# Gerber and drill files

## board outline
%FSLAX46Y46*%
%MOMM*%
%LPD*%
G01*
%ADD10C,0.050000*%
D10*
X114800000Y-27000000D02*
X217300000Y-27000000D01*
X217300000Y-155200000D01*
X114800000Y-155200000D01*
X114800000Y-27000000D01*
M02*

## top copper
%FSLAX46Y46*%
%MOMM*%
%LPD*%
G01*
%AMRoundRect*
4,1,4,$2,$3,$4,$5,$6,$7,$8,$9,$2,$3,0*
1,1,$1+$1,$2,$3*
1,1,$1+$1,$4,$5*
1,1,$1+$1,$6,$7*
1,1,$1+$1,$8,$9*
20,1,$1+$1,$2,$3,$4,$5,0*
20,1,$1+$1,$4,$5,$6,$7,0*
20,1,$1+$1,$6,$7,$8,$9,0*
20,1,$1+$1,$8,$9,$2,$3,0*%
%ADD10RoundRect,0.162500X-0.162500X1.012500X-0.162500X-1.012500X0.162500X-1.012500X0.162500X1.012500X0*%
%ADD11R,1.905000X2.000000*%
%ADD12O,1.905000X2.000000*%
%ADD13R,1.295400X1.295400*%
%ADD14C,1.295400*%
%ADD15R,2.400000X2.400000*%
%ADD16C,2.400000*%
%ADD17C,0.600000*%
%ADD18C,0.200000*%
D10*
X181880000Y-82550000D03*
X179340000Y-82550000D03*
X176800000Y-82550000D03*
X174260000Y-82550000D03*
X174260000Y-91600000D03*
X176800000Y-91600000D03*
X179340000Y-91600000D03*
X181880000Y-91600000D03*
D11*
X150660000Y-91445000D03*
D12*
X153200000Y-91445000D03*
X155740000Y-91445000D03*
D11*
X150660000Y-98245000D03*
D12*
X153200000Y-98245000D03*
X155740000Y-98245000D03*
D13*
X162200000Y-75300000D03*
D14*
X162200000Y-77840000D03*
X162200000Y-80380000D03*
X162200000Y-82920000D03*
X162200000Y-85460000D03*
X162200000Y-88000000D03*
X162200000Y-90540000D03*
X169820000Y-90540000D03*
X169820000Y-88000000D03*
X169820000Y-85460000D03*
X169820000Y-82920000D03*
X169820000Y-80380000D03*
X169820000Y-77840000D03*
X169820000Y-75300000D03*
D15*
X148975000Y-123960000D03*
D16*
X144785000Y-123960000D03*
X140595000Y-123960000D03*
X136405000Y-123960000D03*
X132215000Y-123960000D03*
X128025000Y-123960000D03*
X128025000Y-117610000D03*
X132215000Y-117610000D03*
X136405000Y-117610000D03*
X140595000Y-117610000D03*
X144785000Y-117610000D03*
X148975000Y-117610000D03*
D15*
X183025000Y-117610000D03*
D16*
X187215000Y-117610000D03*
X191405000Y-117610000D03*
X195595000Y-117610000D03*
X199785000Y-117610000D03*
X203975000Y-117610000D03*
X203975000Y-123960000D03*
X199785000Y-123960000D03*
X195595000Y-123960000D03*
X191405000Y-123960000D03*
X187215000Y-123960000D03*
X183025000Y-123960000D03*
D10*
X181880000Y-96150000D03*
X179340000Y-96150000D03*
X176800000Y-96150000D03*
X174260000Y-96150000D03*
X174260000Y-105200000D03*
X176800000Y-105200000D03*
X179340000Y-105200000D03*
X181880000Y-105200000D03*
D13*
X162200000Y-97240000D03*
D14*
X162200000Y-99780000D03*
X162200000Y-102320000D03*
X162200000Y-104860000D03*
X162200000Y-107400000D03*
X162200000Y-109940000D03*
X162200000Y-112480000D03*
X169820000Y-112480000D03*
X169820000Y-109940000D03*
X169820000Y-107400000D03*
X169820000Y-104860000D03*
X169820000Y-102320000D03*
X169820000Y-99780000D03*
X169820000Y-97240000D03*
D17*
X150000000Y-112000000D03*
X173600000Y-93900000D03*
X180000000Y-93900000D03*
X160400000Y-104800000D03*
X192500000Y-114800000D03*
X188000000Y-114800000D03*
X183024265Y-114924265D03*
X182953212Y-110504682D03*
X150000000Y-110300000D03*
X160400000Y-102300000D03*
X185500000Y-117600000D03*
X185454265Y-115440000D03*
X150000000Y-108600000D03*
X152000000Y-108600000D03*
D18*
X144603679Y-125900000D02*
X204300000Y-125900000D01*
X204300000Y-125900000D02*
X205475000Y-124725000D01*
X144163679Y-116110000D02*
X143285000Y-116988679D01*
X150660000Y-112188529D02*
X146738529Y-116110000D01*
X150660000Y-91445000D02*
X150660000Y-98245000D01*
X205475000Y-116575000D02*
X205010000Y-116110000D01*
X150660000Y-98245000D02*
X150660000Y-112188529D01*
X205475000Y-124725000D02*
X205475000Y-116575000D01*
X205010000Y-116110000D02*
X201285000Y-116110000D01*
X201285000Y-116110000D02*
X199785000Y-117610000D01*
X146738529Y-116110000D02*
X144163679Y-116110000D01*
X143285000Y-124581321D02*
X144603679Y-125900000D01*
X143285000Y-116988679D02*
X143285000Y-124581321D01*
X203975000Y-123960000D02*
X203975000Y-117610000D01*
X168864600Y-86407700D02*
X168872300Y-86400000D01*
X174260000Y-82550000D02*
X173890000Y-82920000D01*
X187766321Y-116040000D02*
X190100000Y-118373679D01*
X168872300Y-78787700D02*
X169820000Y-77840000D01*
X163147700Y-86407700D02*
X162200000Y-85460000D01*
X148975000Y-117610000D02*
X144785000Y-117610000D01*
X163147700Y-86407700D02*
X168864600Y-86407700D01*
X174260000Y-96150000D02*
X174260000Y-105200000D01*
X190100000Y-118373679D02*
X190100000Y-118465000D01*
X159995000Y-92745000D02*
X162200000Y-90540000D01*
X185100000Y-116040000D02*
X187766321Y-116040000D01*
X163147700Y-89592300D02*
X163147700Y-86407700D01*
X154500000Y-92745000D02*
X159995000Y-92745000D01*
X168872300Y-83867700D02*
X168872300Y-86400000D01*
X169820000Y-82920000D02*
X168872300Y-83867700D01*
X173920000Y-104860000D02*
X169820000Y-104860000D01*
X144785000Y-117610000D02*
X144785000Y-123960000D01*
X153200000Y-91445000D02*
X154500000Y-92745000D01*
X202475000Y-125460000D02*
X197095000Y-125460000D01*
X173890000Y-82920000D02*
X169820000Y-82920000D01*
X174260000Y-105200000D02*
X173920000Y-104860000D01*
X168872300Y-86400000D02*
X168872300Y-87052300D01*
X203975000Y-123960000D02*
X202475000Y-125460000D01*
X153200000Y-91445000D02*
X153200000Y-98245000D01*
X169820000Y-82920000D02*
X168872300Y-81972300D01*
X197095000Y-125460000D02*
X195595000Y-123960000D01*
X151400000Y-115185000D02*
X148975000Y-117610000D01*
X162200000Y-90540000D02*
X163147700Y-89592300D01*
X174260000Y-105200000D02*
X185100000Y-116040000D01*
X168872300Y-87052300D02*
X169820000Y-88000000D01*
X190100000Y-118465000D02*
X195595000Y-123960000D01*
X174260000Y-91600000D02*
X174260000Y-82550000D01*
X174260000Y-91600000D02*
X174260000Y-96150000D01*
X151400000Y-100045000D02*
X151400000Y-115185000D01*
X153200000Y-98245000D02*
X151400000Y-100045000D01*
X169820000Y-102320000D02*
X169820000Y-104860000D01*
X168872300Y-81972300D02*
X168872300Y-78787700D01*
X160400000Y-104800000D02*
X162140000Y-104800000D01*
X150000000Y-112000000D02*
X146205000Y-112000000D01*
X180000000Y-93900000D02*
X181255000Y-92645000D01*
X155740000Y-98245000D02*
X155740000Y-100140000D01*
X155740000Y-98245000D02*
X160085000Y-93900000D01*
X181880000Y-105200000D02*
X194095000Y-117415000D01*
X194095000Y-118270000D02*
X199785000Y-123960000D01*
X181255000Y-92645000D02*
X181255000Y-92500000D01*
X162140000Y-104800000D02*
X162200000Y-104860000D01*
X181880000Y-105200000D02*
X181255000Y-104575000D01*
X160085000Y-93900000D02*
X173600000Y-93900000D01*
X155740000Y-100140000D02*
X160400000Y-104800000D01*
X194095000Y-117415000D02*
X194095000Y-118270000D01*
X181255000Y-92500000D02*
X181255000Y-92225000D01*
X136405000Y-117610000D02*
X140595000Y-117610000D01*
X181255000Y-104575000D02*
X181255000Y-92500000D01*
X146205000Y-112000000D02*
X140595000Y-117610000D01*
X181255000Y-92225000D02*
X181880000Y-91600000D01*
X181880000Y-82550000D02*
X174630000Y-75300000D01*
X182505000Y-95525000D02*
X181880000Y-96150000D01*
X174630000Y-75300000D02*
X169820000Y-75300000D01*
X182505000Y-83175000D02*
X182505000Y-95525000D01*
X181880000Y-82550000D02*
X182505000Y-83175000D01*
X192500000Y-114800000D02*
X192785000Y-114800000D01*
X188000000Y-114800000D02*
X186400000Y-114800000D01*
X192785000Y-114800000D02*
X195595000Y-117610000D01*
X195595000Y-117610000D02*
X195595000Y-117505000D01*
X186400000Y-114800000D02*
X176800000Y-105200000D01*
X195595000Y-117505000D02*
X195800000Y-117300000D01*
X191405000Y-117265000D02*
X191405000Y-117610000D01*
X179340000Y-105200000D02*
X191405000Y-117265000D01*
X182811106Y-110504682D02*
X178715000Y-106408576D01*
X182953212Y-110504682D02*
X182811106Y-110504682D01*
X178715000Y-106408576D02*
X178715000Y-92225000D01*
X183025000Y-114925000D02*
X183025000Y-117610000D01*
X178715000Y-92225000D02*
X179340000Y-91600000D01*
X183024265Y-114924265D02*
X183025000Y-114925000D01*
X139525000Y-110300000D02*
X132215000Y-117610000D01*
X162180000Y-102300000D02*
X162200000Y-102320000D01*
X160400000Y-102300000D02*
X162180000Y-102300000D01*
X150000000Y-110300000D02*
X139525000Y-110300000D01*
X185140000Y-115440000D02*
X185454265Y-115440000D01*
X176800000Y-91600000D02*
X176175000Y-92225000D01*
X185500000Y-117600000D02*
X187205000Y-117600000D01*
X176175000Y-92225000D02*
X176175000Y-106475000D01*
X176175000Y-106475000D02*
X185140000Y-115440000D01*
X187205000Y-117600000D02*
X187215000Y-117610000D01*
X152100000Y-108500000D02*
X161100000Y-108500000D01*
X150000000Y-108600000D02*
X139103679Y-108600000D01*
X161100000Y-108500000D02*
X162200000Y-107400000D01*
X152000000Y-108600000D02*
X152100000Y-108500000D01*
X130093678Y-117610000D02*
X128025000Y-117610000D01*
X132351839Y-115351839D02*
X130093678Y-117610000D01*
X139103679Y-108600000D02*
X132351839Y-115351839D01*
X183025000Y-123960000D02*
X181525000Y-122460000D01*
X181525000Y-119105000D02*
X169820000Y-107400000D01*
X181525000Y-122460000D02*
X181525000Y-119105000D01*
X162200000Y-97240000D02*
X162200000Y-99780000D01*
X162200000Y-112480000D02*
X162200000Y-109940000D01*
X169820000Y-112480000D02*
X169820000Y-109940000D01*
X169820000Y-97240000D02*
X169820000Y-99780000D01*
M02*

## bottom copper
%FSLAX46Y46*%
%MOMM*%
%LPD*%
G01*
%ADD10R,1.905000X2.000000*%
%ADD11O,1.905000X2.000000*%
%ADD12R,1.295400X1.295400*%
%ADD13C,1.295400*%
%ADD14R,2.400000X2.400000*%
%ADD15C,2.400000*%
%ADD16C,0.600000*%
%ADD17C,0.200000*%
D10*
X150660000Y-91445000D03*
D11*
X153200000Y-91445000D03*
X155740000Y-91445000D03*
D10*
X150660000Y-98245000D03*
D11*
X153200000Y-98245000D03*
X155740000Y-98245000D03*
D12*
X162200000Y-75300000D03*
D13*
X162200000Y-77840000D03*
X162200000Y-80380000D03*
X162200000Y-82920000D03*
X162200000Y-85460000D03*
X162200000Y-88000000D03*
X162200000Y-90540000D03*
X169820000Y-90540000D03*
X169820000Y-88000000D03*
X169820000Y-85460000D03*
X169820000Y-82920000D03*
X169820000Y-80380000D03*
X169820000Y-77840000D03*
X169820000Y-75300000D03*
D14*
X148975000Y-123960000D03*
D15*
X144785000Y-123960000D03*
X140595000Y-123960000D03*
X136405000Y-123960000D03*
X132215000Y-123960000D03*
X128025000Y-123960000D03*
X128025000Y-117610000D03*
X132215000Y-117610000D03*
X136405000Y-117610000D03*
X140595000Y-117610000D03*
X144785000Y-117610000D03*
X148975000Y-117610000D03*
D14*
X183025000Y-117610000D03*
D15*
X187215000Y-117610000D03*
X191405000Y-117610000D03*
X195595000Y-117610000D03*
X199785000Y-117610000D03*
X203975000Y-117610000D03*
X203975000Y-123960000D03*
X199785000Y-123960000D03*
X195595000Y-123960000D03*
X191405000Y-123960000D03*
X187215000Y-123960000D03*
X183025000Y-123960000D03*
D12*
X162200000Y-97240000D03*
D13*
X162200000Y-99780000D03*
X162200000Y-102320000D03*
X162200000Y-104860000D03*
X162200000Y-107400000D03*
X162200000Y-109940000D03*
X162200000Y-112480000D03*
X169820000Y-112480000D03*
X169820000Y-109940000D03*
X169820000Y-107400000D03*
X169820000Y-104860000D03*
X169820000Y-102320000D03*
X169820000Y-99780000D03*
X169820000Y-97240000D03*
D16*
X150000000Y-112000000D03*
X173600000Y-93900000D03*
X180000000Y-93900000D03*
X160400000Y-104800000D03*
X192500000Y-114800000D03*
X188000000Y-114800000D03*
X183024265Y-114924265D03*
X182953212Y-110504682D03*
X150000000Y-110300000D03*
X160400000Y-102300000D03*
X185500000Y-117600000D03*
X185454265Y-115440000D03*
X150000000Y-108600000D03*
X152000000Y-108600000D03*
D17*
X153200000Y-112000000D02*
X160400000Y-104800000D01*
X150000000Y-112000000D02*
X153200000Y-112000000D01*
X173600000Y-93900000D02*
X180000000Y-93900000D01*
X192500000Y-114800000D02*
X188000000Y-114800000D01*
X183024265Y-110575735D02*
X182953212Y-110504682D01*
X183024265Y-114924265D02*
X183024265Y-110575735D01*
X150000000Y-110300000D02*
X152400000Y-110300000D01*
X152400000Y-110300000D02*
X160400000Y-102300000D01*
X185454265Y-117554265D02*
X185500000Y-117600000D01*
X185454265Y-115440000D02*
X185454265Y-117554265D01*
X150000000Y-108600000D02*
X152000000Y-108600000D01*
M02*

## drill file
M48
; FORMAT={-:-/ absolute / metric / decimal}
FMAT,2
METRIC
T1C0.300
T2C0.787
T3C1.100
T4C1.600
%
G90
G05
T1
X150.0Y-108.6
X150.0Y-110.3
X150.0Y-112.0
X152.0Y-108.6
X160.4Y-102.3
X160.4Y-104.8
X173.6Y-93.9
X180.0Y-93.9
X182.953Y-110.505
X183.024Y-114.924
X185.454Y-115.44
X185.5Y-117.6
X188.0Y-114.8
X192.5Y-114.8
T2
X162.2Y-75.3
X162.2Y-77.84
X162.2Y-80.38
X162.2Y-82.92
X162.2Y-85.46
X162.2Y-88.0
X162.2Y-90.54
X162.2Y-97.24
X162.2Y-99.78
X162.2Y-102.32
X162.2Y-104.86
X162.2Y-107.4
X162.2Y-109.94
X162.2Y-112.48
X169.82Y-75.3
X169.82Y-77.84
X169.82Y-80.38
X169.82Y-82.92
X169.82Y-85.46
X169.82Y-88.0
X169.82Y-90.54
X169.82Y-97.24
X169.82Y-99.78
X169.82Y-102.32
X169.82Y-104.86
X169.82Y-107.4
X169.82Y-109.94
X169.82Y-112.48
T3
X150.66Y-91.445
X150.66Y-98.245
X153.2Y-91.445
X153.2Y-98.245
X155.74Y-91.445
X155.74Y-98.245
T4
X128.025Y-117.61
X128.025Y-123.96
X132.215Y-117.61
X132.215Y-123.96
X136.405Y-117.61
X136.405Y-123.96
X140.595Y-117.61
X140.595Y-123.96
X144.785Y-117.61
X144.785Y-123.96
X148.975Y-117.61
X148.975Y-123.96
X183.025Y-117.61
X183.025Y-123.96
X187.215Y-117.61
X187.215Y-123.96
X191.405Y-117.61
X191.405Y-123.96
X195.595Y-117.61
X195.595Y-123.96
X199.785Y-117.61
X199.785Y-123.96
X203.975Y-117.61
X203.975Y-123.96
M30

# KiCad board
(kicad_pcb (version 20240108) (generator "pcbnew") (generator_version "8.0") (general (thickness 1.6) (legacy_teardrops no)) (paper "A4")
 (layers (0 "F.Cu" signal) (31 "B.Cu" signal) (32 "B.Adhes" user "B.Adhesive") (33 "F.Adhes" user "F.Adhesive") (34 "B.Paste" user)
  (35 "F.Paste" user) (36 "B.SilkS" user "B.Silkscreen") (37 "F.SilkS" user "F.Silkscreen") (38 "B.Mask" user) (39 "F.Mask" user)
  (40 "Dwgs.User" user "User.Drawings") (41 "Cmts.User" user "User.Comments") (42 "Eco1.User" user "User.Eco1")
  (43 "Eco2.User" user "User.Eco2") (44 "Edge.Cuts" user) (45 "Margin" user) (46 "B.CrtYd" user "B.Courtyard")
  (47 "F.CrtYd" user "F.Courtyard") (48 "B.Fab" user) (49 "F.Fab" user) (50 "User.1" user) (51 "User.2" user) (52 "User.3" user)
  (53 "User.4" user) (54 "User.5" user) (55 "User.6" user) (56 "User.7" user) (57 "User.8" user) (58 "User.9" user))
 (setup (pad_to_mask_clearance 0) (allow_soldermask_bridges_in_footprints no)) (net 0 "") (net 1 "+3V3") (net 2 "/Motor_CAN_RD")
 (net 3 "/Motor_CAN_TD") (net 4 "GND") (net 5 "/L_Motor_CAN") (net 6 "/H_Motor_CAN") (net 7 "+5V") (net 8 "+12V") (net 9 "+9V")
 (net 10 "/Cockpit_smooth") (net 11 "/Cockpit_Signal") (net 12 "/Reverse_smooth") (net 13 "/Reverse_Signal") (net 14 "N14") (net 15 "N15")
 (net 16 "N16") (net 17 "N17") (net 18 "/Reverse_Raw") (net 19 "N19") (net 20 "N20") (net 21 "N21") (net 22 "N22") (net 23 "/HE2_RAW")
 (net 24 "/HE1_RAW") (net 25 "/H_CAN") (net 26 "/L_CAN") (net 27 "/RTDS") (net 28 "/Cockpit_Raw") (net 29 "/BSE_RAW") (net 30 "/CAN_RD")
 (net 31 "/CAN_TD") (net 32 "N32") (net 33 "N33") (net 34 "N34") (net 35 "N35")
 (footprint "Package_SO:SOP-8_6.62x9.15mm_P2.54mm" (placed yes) (layer "F.Cu") (at 178.07 87.075 -90)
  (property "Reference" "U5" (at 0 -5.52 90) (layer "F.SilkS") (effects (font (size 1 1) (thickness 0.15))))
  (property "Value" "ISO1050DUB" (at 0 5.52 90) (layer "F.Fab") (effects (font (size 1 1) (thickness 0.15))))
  (pad "1" smd roundrect (at -4.525 -3.81 270) (size 2.35 0.65) (layers "F.Cu" "F.Paste" "F.Mask") (roundrect_rratio 0.25) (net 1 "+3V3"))
  (pad "2" smd roundrect (at -4.525 -1.27 270) (size 2.35 0.65) (layers "F.Cu" "F.Paste" "F.Mask") (roundrect_rratio 0.25)
   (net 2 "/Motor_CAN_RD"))
  (pad "3" smd roundrect (at -4.525 1.27 270) (size 2.35 0.65) (layers "F.Cu" "F.Paste" "F.Mask") (roundrect_rratio 0.25)
   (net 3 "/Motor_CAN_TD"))
  (pad "4" smd roundrect (at -4.525 3.81 270) (size 2.35 0.65) (layers "F.Cu" "F.Paste" "F.Mask") (roundrect_rratio 0.25) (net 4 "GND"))
  (pad "5" smd roundrect (at 4.525 3.81 270) (size 2.35 0.65) (layers "F.Cu" "F.Paste" "F.Mask") (roundrect_rratio 0.25) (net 4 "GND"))
  (pad "6" smd roundrect (at 4.525 1.27 270) (size 2.35 0.65) (layers "F.Cu" "F.Paste" "F.Mask") (roundrect_rratio 0.25)
   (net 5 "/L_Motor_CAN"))
  (pad "7" smd roundrect (at 4.525 -1.27 270) (size 2.35 0.65) (layers "F.Cu" "F.Paste" "F.Mask") (roundrect_rratio 0.25)
   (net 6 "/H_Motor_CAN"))
  (pad "8" smd roundrect (at 4.525 -3.81 270) (size 2.35 0.65) (layers "F.Cu" "F.Paste" "F.Mask") (roundrect_rratio 0.25) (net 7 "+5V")))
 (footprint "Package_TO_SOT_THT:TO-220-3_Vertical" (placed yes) (layer "F.Cu") (at 150.66 91.445)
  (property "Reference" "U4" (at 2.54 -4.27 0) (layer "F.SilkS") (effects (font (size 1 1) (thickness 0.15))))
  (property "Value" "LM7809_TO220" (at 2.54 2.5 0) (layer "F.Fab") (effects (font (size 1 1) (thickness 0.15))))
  (pad "1" thru_hole rect (at 0 0) (size 1.905 2) (drill 1.1) (layers "*.Cu" "*.Mask") (remove_unused_layers no) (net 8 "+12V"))
  (pad "2" thru_hole oval (at 2.54 0) (size 1.905 2) (drill 1.1) (layers "*.Cu" "*.Mask") (remove_unused_layers no) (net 4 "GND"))
  (pad "3" thru_hole oval (at 5.08 0) (size 1.905 2) (drill 1.1) (layers "*.Cu" "*.Mask") (remove_unused_layers no) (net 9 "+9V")))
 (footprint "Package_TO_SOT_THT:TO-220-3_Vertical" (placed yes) (layer "F.Cu") (at 150.66 98.245)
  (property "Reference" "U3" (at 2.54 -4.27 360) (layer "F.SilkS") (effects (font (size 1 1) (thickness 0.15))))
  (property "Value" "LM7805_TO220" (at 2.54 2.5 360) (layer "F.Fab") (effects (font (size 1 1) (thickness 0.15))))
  (pad "1" thru_hole rect (at 0 0) (size 1.905 2) (drill 1.1) (layers "*.Cu" "*.Mask") (remove_unused_layers no) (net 8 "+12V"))
  (pad "2" thru_hole oval (at 2.54 0) (size 1.905 2) (drill 1.1) (layers "*.Cu" "*.Mask") (remove_unused_layers no) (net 4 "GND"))
  (pad "3" thru_hole oval (at 5.08 0) (size 1.905 2) (drill 1.1) (layers "*.Cu" "*.Mask") (remove_unused_layers no) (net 7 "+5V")))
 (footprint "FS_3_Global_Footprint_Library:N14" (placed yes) (layer "F.Cu") (at 169.82 90.54)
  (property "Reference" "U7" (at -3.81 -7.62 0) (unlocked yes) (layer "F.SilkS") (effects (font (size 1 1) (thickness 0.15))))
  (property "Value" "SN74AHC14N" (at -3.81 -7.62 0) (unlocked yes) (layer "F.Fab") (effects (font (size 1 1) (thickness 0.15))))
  (pad "1" thru_hole rect (at -7.62 -15.24) (size 1.2954 1.2954) (drill 0.7874) (layers "*.Cu" "*.Mask") (remove_unused_layers no)
   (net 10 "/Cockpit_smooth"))
  (pad "2" thru_hole circle (at -7.62 -12.7) (size 1.2954 1.2954) (drill 0.7874) (layers "*.Cu" "*.Mask") (remove_unused_layers no)
   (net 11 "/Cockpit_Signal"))
  (pad "3" thru_hole circle (at -7.62 -10.16) (size 1.2954 1.2954) (drill 0.7874) (layers "*.Cu" "*.Mask") (remove_unused_layers no)
   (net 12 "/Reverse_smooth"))
  (pad "4" thru_hole circle (at -7.62 -7.62) (size 1.2954 1.2954) (drill 0.7874) (layers "*.Cu" "*.Mask") (remove_unused_layers no)
   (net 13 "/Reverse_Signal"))
  (pad "5" thru_hole circle (at -7.62 -5.08) (size 1.2954 1.2954) (drill 0.7874) (layers "*.Cu" "*.Mask") (remove_unused_layers no)
   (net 4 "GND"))
  (pad "6" thru_hole circle (at -7.62 -2.54) (size 1.2954 1.2954) (drill 0.7874) (layers "*.Cu" "*.Mask") (remove_unused_layers no)
   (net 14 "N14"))
  (pad "7" thru_hole circle (at -7.62 0) (size 1.2954 1.2954) (drill 0.7874) (layers "*.Cu" "*.Mask") (remove_unused_layers no)
   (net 4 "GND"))
  (pad "8" thru_hole circle (at 0 0) (size 1.2954 1.2954) (drill 0.7874) (layers "*.Cu" "*.Mask") (remove_unused_layers no) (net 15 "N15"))
  (pad "9" thru_hole circle (at 0 -2.54) (size 1.2954 1.2954) (drill 0.7874) (layers "*.Cu" "*.Mask") (remove_unused_layers no)
   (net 4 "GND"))
  (pad "10" thru_hole circle (at 0 -5.08) (size 1.2954 1.2954) (drill 0.7874) (layers "*.Cu" "*.Mask") (remove_unused_layers no)
   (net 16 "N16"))
  (pad "11" thru_hole circle (at 0 -7.62) (size 1.2954 1.2954) (drill 0.7874) (layers "*.Cu" "*.Mask") (remove_unused_layers no)
   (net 4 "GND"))
  (pad "12" thru_hole circle (at 0 -10.16) (size 1.2954 1.2954) (drill 0.7874) (layers "*.Cu" "*.Mask") (remove_unused_layers no)
   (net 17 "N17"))
  (pad "13" thru_hole circle (at 0 -12.7) (size 1.2954 1.2954) (drill 0.7874) (layers "*.Cu" "*.Mask") (remove_unused_layers no)
   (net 4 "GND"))
  (pad "14" thru_hole circle (at 0 -15.24) (size 1.2954 1.2954) (drill 0.7874) (layers "*.Cu" "*.Mask") (remove_unused_layers no)
   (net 1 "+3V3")))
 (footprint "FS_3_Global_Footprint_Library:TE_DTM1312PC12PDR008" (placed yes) (layer "F.Cu") (at 166 122)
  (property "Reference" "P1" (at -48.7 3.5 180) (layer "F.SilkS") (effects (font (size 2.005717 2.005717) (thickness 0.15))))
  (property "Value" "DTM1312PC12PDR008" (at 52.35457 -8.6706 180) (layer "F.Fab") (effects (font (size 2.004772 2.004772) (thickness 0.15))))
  (pad "C1" thru_hole rect (at -17.025 1.96) (size 2.4 2.4) (drill 1.6) (layers "*.Cu" "*.Mask") (remove_unused_layers no)
   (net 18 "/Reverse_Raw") (solder_mask_margin 0.102))
  (pad "C2" thru_hole circle (at -21.215 1.96) (size 2.4 2.4) (drill 1.6) (layers "*.Cu" "*.Mask") (remove_unused_layers no) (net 4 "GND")
   (solder_mask_margin 0.102))
  (pad "C3" thru_hole circle (at -25.405 1.96) (size 2.4 2.4) (drill 1.6) (layers "*.Cu" "*.Mask") (remove_unused_layers no) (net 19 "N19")
   (solder_mask_margin 0.102))
  (pad "C4" thru_hole circle (at -29.595 1.96) (size 2.4 2.4) (drill 1.6) (layers "*.Cu" "*.Mask") (remove_unused_layers no) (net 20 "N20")
   (solder_mask_margin 0.102))
  (pad "C5" thru_hole circle (at -33.785 1.96) (size 2.4 2.4) (drill 1.6) (layers "*.Cu" "*.Mask") (remove_unused_layers no) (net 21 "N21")
   (solder_mask_margin 0.102))
  (pad "C6" thru_hole circle (at -37.975 1.96) (size 2.4 2.4) (drill 1.6) (layers "*.Cu" "*.Mask") (remove_unused_layers no) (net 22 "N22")
   (solder_mask_margin 0.102))
  (pad "C7" thru_hole circle (at -37.975 -4.39) (size 2.4 2.4) (drill 1.6) (layers "*.Cu" "*.Mask") (remove_unused_layers no)
   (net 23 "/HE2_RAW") (solder_mask_margin 0.102))
  (pad "C8" thru_hole circle (at -33.785 -4.39) (size 2.4 2.4) (drill 1.6) (layers "*.Cu" "*.Mask") (remove_unused_layers no)
   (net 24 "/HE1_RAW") (solder_mask_margin 0.102))
  (pad "C9" thru_hole circle (at -29.595 -4.39) (size 2.4 2.4) (drill 1.6) (layers "*.Cu" "*.Mask") (remove_unused_layers no) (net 7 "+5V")
   (solder_mask_margin 0.102))
  (pad "C10" thru_hole circle (at -25.405 -4.39) (size 2.4 2.4) (drill 1.6) (layers "*.Cu" "*.Mask") (remove_unused_layers no) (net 7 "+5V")
   (solder_mask_margin 0.102))
  (pad "C11" thru_hole circle (at -21.215 -4.39) (size 2.4 2.4) (drill 1.6) (layers "*.Cu" "*.Mask") (remove_unused_layers no) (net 4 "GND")
   (solder_mask_margin 0.102))
  (pad "C12" thru_hole circle (at -17.025 -4.39) (size 2.4 2.4) (drill 1.6) (layers "*.Cu" "*.Mask") (remove_unused_layers no) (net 4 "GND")
   (solder_mask_margin 0.102))
  (pad "D1" thru_hole rect (at 17.025 -4.39) (size 2.4 2.4) (drill 1.6) (layers "*.Cu" "*.Mask") (remove_unused_layers no)
   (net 6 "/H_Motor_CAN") (solder_mask_margin 0.102))
  (pad "D2" thru_hole circle (at 21.215 -4.39) (size 2.4 2.4) (drill 1.6) (layers "*.Cu" "*.Mask") (remove_unused_layers no)
   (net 5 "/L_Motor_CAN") (solder_mask_margin 0.102))
  (pad "D3" thru_hole circle (at 25.405 -4.39) (size 2.4 2.4) (drill 1.6) (layers "*.Cu" "*.Mask") (remove_unused_layers no)
   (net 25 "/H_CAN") (solder_mask_margin 0.102))
  (pad "D4" thru_hole circle (at 29.595 -4.39) (size 2.4 2.4) (drill 1.6) (layers "*.Cu" "*.Mask") (remove_unused_layers no)
   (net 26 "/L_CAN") (solder_mask_margin 0.102))
  (pad "D5" thru_hole circle (at 33.785 -4.39) (size 2.4 2.4) (drill 1.6) (layers "*.Cu" "*.Mask") (remove_unused_layers no) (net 8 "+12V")
   (solder_mask_margin 0.102))
  (pad "D6" thru_hole circle (at 37.975 -4.39) (size 2.4 2.4) (drill 1.6) (layers "*.Cu" "*.Mask") (remove_unused_layers no) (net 4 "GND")
   (solder_mask_margin 0.102))
  (pad "D7" thru_hole circle (at 37.975 1.96) (size 2.4 2.4) (drill 1.6) (layers "*.Cu" "*.Mask") (remove_unused_layers no) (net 4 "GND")
   (solder_mask_margin 0.102))
  (pad "D8" thru_hole circle (at 33.785 1.96) (size 2.4 2.4) (drill 1.6) (layers "*.Cu" "*.Mask") (remove_unused_layers no) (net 7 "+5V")
   (solder_mask_margin 0.102))
  (pad "D9" thru_hole circle (at 29.595 1.96) (size 2.4 2.4) (drill 1.6) (layers "*.Cu" "*.Mask") (remove_unused_layers no) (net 4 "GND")
   (solder_mask_margin 0.102))
  (pad "D10" thru_hole circle (at 25.405 1.96) (size 2.4 2.4) (drill 1.6) (layers "*.Cu" "*.Mask") (remove_unused_layers no)
   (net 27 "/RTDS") (solder_mask_margin 0.102))
  (pad "D11" thru_hole circle (at 21.215 1.96) (size 2.4 2.4) (drill 1.6) (layers "*.Cu" "*.Mask") (remove_unused_layers no)
   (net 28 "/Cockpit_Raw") (solder_mask_margin 0.102))
  (pad "D12" thru_hole circle (at 17.025 1.96) (size 2.4 2.4) (drill 1.6) (layers "*.Cu" "*.Mask") (remove_unused_layers no)
   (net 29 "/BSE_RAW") (solder_mask_margin 0.102)))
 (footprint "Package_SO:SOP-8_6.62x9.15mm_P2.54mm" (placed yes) (layer "F.Cu") (at 178.07 100.675 -90)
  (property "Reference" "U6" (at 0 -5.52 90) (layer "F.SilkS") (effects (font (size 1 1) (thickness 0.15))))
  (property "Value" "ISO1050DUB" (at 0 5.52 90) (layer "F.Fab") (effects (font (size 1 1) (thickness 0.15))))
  (pad "1" smd roundrect (at -4.525 -3.81 270) (size 2.35 0.65) (layers "F.Cu" "F.Paste" "F.Mask") (roundrect_rratio 0.25) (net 1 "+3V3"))
  (pad "2" smd roundrect (at -4.525 -1.27 270) (size 2.35 0.65) (layers "F.Cu" "F.Paste" "F.Mask") (roundrect_rratio 0.25)
   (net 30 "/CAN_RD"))
  (pad "3" smd roundrect (at -4.525 1.27 270) (size 2.35 0.65) (layers "F.Cu" "F.Paste" "F.Mask") (roundrect_rratio 0.25) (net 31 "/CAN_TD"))
  (pad "4" smd roundrect (at -4.525 3.81 270) (size 2.35 0.65) (layers "F.Cu" "F.Paste" "F.Mask") (roundrect_rratio 0.25) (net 4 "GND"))
  (pad "5" smd roundrect (at 4.525 3.81 270) (size 2.35 0.65) (layers "F.Cu" "F.Paste" "F.Mask") (roundrect_rratio 0.25) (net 4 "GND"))
  (pad "6" smd roundrect (at 4.525 1.27 270) (size 2.35 0.65) (layers "F.Cu" "F.Paste" "F.Mask") (roundrect_rratio 0.25) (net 26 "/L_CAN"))
  (pad "7" smd roundrect (at 4.525 -1.27 270) (size 2.35 0.65) (layers "F.Cu" "F.Paste" "F.Mask") (roundrect_rratio 0.25) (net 25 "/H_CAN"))
  (pad "8" smd roundrect (at 4.525 -3.81 270) (size 2.35 0.65) (layers "F.Cu" "F.Paste" "F.Mask") (roundrect_rratio 0.25) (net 7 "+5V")))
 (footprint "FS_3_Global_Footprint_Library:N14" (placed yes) (layer "F.Cu") (at 169.82 112.48)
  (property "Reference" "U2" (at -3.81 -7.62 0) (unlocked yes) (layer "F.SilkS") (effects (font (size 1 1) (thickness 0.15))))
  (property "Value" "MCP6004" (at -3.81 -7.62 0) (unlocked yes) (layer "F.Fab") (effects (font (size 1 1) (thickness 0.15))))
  (pad "1" thru_hole rect (at -7.62 -15.24) (size 1.2954 1.2954) (drill 0.7874) (layers "*.Cu" "*.Mask") (remove_unused_layers no)
   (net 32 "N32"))
  (pad "2" thru_hole circle (at -7.62 -12.7) (size 1.2954 1.2954) (drill 0.7874) (layers "*.Cu" "*.Mask") (remove_unused_layers no)
   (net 32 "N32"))
  (pad "3" thru_hole circle (at -7.62 -10.16) (size 1.2954 1.2954) (drill 0.7874) (layers "*.Cu" "*.Mask") (remove_unused_layers no)
   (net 24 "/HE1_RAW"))
  (pad "4" thru_hole circle (at -7.62 -7.62) (size 1.2954 1.2954) (drill 0.7874) (layers "*.Cu" "*.Mask") (remove_unused_layers no)
   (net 7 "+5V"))
  (pad "5" thru_hole circle (at -7.62 -5.08) (size 1.2954 1.2954) (drill 0.7874) (layers "*.Cu" "*.Mask") (remove_unused_layers no)
   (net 23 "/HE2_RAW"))
  (pad "6" thru_hole circle (at -7.62 -2.54) (size 1.2954 1.2954) (drill 0.7874) (layers "*.Cu" "*.Mask") (remove_unused_layers no)
   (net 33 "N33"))
  (pad "7" thru_hole circle (at -7.62 0) (size 1.2954 1.2954) (drill 0.7874) (layers "*.Cu" "*.Mask") (remove_unused_layers no)
   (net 33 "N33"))
  (pad "8" thru_hole circle (at 0 0) (size 1.2954 1.2954) (drill 0.7874) (layers "*.Cu" "*.Mask") (remove_unused_layers no) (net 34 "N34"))
  (pad "9" thru_hole circle (at 0 -2.54) (size 1.2954 1.2954) (drill 0.7874) (layers "*.Cu" "*.Mask") (remove_unused_layers no)
   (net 34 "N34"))
  (pad "10" thru_hole circle (at 0 -5.08) (size 1.2954 1.2954) (drill 0.7874) (layers "*.Cu" "*.Mask") (remove_unused_layers no)
   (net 29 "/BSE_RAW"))
  (pad "11" thru_hole circle (at 0 -7.62) (size 1.2954 1.2954) (drill 0.7874) (layers "*.Cu" "*.Mask") (remove_unused_layers no)
   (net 4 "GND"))
  (pad "12" thru_hole circle (at 0 -10.16) (size 1.2954 1.2954) (drill 0.7874) (layers "*.Cu" "*.Mask") (remove_unused_layers no)
   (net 4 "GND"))
  (pad "13" thru_hole circle (at 0 -12.7) (size 1.2954 1.2954) (drill 0.7874) (layers "*.Cu" "*.Mask") (remove_unused_layers no)
   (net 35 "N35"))
  (pad "14" thru_hole circle (at 0 -15.24) (size 1.2954 1.2954) (drill 0.7874) (layers "*.Cu" "*.Mask") (remove_unused_layers no)
   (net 35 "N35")))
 (gr_rect (start 114.8 27) (end 217.3 155.2) (stroke (width 0.05) (type default)) (fill none) (layer "Edge.Cuts"))
 (segment (start 144.603679 125.9) (end 204.3 125.9) (width 0.2) (layer "F.Cu") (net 8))
 (segment (start 204.3 125.9) (end 205.475 124.725) (width 0.2) (layer "F.Cu") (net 8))
 (segment (start 144.163679 116.11) (end 143.285 116.988679) (width 0.2) (layer "F.Cu") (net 8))
 (segment (start 150.66 112.188529) (end 146.738529 116.11) (width 0.2) (layer "F.Cu") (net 8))
 (segment (start 150.66 91.445) (end 150.66 98.245) (width 0.2) (layer "F.Cu") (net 8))
 (segment (start 205.475 116.575) (end 205.01 116.11) (width 0.2) (layer "F.Cu") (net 8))
 (segment (start 150.66 98.245) (end 150.66 112.188529) (width 0.2) (layer "F.Cu") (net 8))
 (segment (start 205.475 124.725) (end 205.475 116.575) (width 0.2) (layer "F.Cu") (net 8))
 (segment (start 205.01 116.11) (end 201.285 116.11) (width 0.2) (layer "F.Cu") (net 8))
 (segment (start 201.285 116.11) (end 199.785 117.61) (width 0.2) (layer "F.Cu") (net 8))
 (segment (start 146.738529 116.11) (end 144.163679 116.11) (width 0.2) (layer "F.Cu") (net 8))
 (segment (start 143.285 124.581321) (end 144.603679 125.9) (width 0.2) (layer "F.Cu") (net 8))
 (segment (start 143.285 116.988679) (end 143.285 124.581321) (width 0.2) (layer "F.Cu") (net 8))
 (segment (start 203.975 123.96) (end 203.975 117.61) (width 0.2) (layer "F.Cu") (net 4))
 (segment (start 168.8646 86.4077) (end 168.8723 86.4) (width 0.2) (layer "F.Cu") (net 4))
 (segment (start 174.26 82.55) (end 173.89 82.92) (width 0.2) (layer "F.Cu") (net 4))
 (segment (start 187.766321 116.04) (end 190.1 118.373679) (width 0.2) (layer "F.Cu") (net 4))
 (segment (start 168.8723 78.7877) (end 169.82 77.84) (width 0.2) (layer "F.Cu") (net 4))
 (segment (start 163.1477 86.4077) (end 162.2 85.46) (width 0.2) (layer "F.Cu") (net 4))
 (segment (start 148.975 117.61) (end 144.785 117.61) (width 0.2) (layer "F.Cu") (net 4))
 (segment (start 163.1477 86.4077) (end 168.8646 86.4077) (width 0.2) (layer "F.Cu") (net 4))
 (segment (start 174.26 96.15) (end 174.26 105.2) (width 0.2) (layer "F.Cu") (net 4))
 (segment (start 190.1 118.373679) (end 190.1 118.465) (width 0.2) (layer "F.Cu") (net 4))
 (segment (start 159.995 92.745) (end 162.2 90.54) (width 0.2) (layer "F.Cu") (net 4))
 (segment (start 185.1 116.04) (end 187.766321 116.04) (width 0.2) (layer "F.Cu") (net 4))
 (segment (start 163.1477 89.5923) (end 163.1477 86.4077) (width 0.2) (layer "F.Cu") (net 4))
 (segment (start 154.5 92.745) (end 159.995 92.745) (width 0.2) (layer "F.Cu") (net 4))
 (segment (start 168.8723 83.8677) (end 168.8723 86.4) (width 0.2) (layer "F.Cu") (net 4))
 (segment (start 169.82 82.92) (end 168.8723 83.8677) (width 0.2) (layer "F.Cu") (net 4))
 (segment (start 173.92 104.86) (end 169.82 104.86) (width 0.2) (layer "F.Cu") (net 4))
 (segment (start 144.785 117.61) (end 144.785 123.96) (width 0.2) (layer "F.Cu") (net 4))
 (segment (start 153.2 91.445) (end 154.5 92.745) (width 0.2) (layer "F.Cu") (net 4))
 (segment (start 202.475 125.46) (end 197.095 125.46) (width 0.2) (layer "F.Cu") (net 4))
 (segment (start 173.89 82.92) (end 169.82 82.92) (width 0.2) (layer "F.Cu") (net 4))
 (segment (start 174.26 105.2) (end 173.92 104.86) (width 0.2) (layer "F.Cu") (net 4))
 (segment (start 168.8723 86.4) (end 168.8723 87.0523) (width 0.2) (layer "F.Cu") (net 4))
 (segment (start 203.975 123.96) (end 202.475 125.46) (width 0.2) (layer "F.Cu") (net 4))
 (segment (start 153.2 91.445) (end 153.2 98.245) (width 0.2) (layer "F.Cu") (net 4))
 (segment (start 169.82 82.92) (end 168.8723 81.9723) (width 0.2) (layer "F.Cu") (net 4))
 (segment (start 197.095 125.46) (end 195.595 123.96) (width 0.2) (layer "F.Cu") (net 4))
 (segment (start 151.4 115.185) (end 148.975 117.61) (width 0.2) (layer "F.Cu") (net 4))
 (segment (start 162.2 90.54) (end 163.1477 89.5923) (width 0.2) (layer "F.Cu") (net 4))
 (segment (start 174.26 105.2) (end 185.1 116.04) (width 0.2) (layer "F.Cu") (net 4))
 (segment (start 168.8723 87.0523) (end 169.82 88) (width 0.2) (layer "F.Cu") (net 4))
 (segment (start 190.1 118.465) (end 195.595 123.96) (width 0.2) (layer "F.Cu") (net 4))
 (segment (start 174.26 91.6) (end 174.26 82.55) (width 0.2) (layer "F.Cu") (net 4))
 (segment (start 174.26 91.6) (end 174.26 96.15) (width 0.2) (layer "F.Cu") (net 4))
 (segment (start 151.4 100.045) (end 151.4 115.185) (width 0.2) (layer "F.Cu") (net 4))
 (segment (start 153.2 98.245) (end 151.4 100.045) (width 0.2) (layer "F.Cu") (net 4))
 (segment (start 169.82 102.32) (end 169.82 104.86) (width 0.2) (layer "F.Cu") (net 4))
 (segment (start 168.8723 81.9723) (end 168.8723 78.7877) (width 0.2) (layer "F.Cu") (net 4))
 (segment (start 160.4 104.8) (end 162.14 104.8) (width 0.2) (layer "F.Cu") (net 7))
 (segment (start 150 112) (end 146.205 112) (width 0.2) (layer "F.Cu") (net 7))
 (segment (start 180 93.9) (end 181.255 92.645) (width 0.2) (layer "F.Cu") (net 7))
 (segment (start 155.74 98.245) (end 155.74 100.14) (width 0.2) (layer "F.Cu") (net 7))
 (segment (start 155.74 98.245) (end 160.085 93.9) (width 0.2) (layer "F.Cu") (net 7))
 (segment (start 181.88 105.2) (end 194.095 117.415) (width 0.2) (layer "F.Cu") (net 7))
 (segment (start 194.095 118.27) (end 199.785 123.96) (width 0.2) (layer "F.Cu") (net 7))
 (segment (start 181.255 92.645) (end 181.255 92.5) (width 0.2) (layer "F.Cu") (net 7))
 (segment (start 162.14 104.8) (end 162.2 104.86) (width 0.2) (layer "F.Cu") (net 7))
 (segment (start 181.88 105.2) (end 181.255 104.575) (width 0.2) (layer "F.Cu") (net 7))
 (segment (start 160.085 93.9) (end 173.6 93.9) (width 0.2) (layer "F.Cu") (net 7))
 (segment (start 155.74 100.14) (end 160.4 104.8) (width 0.2) (layer "F.Cu") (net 7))
 (segment (start 194.095 117.415) (end 194.095 118.27) (width 0.2) (layer "F.Cu") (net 7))
 (segment (start 181.255 92.5) (end 181.255 92.225) (width 0.2) (layer "F.Cu") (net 7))
 (segment (start 136.405 117.61) (end 140.595 117.61) (width 0.2) (layer "F.Cu") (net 7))
 (segment (start 181.255 104.575) (end 181.255 92.5) (width 0.2) (layer "F.Cu") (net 7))
 (segment (start 146.205 112) (end 140.595 117.61) (width 0.2) (layer "F.Cu") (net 7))
 (segment (start 181.255 92.225) (end 181.88 91.6) (width 0.2) (layer "F.Cu") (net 7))
 (via (at 150 112) (size 0.6) (drill 0.3) (layers "F.Cu" "B.Cu") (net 7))
 (via (at 173.6 93.9) (size 0.6) (drill 0.3) (layers "F.Cu" "B.Cu") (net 7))
 (via (at 180 93.9) (size 0.6) (drill 0.3) (layers "F.Cu" "B.Cu") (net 7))
 (via (at 160.4 104.8) (size 0.6) (drill 0.3) (layers "F.Cu" "B.Cu") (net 7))
 (segment (start 153.2 112) (end 160.4 104.8) (width 0.2) (layer "B.Cu") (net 7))
 (segment (start 150 112) (end 153.2 112) (width 0.2) (layer "B.Cu") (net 7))
 (segment (start 173.6 93.9) (end 180 93.9) (width 0.2) (layer "B.Cu") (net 7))
 (segment (start 181.88 82.55) (end 174.63 75.3) (width 0.2) (layer "F.Cu") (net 1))
 (segment (start 182.505 95.525) (end 181.88 96.15) (width 0.2) (layer "F.Cu") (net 1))
 (segment (start 174.63 75.3) (end 169.82 75.3) (width 0.2) (layer "F.Cu") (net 1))
 (segment (start 182.505 83.175) (end 182.505 95.525) (width 0.2) (layer "F.Cu") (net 1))
 (segment (start 181.88 82.55) (end 182.505 83.175) (width 0.2) (layer "F.Cu") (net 1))
 (segment (start 192.5 114.8) (end 192.785 114.8) (width 0.2) (layer "F.Cu") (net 26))
 (segment (start 188 114.8) (end 186.4 114.8) (width 0.2) (layer "F.Cu") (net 26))
 (segment (start 192.785 114.8) (end 195.595 117.61) (width 0.2) (layer "F.Cu") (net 26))
 (segment (start 195.595 117.61) (end 195.595 117.505) (width 0.2) (layer "F.Cu") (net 26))
 (segment (start 186.4 114.8) (end 176.8 105.2) (width 0.2) (layer "F.Cu") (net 26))
 (segment (start 195.595 117.505) (end 195.8 117.3) (width 0.2) (layer "F.Cu") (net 26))
 (via (at 192.5 114.8) (size 0.6) (drill 0.3) (layers "F.Cu" "B.Cu") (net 26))
 (via (at 188 114.8) (size 0.6) (drill 0.3) (layers "F.Cu" "B.Cu") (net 26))
 (segment (start 192.5 114.8) (end 188 114.8) (width 0.2) (layer "B.Cu") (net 26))
 (segment (start 191.405 117.265) (end 191.405 117.61) (width 0.2) (layer "F.Cu") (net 25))
 (segment (start 179.34 105.2) (end 191.405 117.265) (width 0.2) (layer "F.Cu") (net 25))
 (segment (start 182.811106 110.504682) (end 178.715 106.408576) (width 0.2) (layer "F.Cu") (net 6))
 (segment (start 182.953212 110.504682) (end 182.811106 110.504682) (width 0.2) (layer "F.Cu") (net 6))
 (segment (start 178.715 106.408576) (end 178.715 92.225) (width 0.2) (layer "F.Cu") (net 6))
 (segment (start 183.025 114.925) (end 183.025 117.61) (width 0.2) (layer "F.Cu") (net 6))
 (segment (start 178.715 92.225) (end 179.34 91.6) (width 0.2) (layer "F.Cu") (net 6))
 (segment (start 183.024265 114.924265) (end 183.025 114.925) (width 0.2) (layer "F.Cu") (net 6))
 (via (at 183.024265 114.924265) (size 0.6) (drill 0.3) (layers "F.Cu" "B.Cu") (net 6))
 (via (at 182.953212 110.504682) (size 0.6) (drill 0.3) (layers "F.Cu" "B.Cu") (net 6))
 (segment (start 183.024265 110.575735) (end 182.953212 110.504682) (width 0.2) (layer "B.Cu") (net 6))
 (segment (start 183.024265 114.924265) (end 183.024265 110.575735) (width 0.2) (layer "B.Cu") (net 6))
 (segment (start 139.525 110.3) (end 132.215 117.61) (width 0.2) (layer "F.Cu") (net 24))
 (segment (start 162.18 102.3) (end 162.2 102.32) (width 0.2) (layer "F.Cu") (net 24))
 (segment (start 160.4 102.3) (end 162.18 102.3) (width 0.2) (layer "F.Cu") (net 24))
 (segment (start 150 110.3) (end 139.525 110.3) (width 0.2) (layer "F.Cu") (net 24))
 (via (at 150 110.3) (size 0.6) (drill 0.3) (layers "F.Cu" "B.Cu") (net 24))
 (via (at 160.4 102.3) (size 0.6) (drill 0.3) (layers "F.Cu" "B.Cu") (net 24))
 (segment (start 150 110.3) (end 152.4 110.3) (width 0.2) (layer "B.Cu") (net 24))
 (segment (start 152.4 110.3) (end 160.4 102.3) (width 0.2) (layer "B.Cu") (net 24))
 (segment (start 185.14 115.44) (end 185.454265 115.44) (width 0.2) (layer "F.Cu") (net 5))
 (segment (start 176.8 91.6) (end 176.175 92.225) (width 0.2) (layer "F.Cu") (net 5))
 (segment (start 185.5 117.6) (end 187.205 117.6) (width 0.2) (layer "F.Cu") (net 5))
 (segment (start 176.175 92.225) (end 176.175 106.475) (width 0.2) (layer "F.Cu") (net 5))
 (segment (start 176.175 106.475) (end 185.14 115.44) (width 0.2) (layer "F.Cu") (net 5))
 (segment (start 187.205 117.6) (end 187.215 117.61) (width 0.2) (layer "F.Cu") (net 5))
 (via (at 185.5 117.6) (size 0.6) (drill 0.3) (layers "F.Cu" "B.Cu") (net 5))
 (via (at 185.454265 115.44) (size 0.6) (drill 0.3) (layers "F.Cu" "B.Cu") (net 5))
 (segment (start 185.454265 117.554265) (end 185.5 117.6) (width 0.2) (layer "B.Cu") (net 5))
 (segment (start 185.454265 115.44) (end 185.454265 117.554265) (width 0.2) (layer "B.Cu") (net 5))
 (segment (start 152.1 108.5) (end 161.1 108.5) (width 0.2) (layer "F.Cu") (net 23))
 (segment (start 150 108.6) (end 139.103679 108.6) (width 0.2) (layer "F.Cu") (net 23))
 (segment (start 161.1 108.5) (end 162.2 107.4) (width 0.2) (layer "F.Cu") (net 23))
 (segment (start 152 108.6) (end 152.1 108.5) (width 0.2) (layer "F.Cu") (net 23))
 (segment (start 130.093678 117.61) (end 128.025 117.61) (width 0.2) (layer "F.Cu") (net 23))
 (segment (start 132.351839 115.351839) (end 130.093678 117.61) (width 0.2) (layer "F.Cu") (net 23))
 (segment (start 139.103679 108.6) (end 132.351839 115.351839) (width 0.2) (layer "F.Cu") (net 23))
 (via (at 150 108.6) (size 0.6) (drill 0.3) (layers "F.Cu" "B.Cu") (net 23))
 (via (at 152 108.6) (size 0.6) (drill 0.3) (layers "F.Cu" "B.Cu") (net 23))
 (segment (start 150 108.6) (end 152 108.6) (width 0.2) (layer "B.Cu") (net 23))
 (segment (start 183.025 123.96) (end 181.525 122.46) (width 0.2) (layer "F.Cu") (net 29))
 (segment (start 181.525 119.105) (end 169.82 107.4) (width 0.2) (layer "F.Cu") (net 29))
 (segment (start 181.525 122.46) (end 181.525 119.105) (width 0.2) (layer "F.Cu") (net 29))
 (segment (start 162.2 97.24) (end 162.2 99.78) (width 0.2) (layer "F.Cu") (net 32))
 (segment (start 162.2 112.48) (end 162.2 109.94) (width 0.2) (layer "F.Cu") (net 33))
 (segment (start 169.82 112.48) (end 169.82 109.94) (width 0.2) (layer "F.Cu") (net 34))
 (segment (start 169.82 97.24) (end 169.82 99.78) (width 0.2) (layer "F.Cu") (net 35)))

